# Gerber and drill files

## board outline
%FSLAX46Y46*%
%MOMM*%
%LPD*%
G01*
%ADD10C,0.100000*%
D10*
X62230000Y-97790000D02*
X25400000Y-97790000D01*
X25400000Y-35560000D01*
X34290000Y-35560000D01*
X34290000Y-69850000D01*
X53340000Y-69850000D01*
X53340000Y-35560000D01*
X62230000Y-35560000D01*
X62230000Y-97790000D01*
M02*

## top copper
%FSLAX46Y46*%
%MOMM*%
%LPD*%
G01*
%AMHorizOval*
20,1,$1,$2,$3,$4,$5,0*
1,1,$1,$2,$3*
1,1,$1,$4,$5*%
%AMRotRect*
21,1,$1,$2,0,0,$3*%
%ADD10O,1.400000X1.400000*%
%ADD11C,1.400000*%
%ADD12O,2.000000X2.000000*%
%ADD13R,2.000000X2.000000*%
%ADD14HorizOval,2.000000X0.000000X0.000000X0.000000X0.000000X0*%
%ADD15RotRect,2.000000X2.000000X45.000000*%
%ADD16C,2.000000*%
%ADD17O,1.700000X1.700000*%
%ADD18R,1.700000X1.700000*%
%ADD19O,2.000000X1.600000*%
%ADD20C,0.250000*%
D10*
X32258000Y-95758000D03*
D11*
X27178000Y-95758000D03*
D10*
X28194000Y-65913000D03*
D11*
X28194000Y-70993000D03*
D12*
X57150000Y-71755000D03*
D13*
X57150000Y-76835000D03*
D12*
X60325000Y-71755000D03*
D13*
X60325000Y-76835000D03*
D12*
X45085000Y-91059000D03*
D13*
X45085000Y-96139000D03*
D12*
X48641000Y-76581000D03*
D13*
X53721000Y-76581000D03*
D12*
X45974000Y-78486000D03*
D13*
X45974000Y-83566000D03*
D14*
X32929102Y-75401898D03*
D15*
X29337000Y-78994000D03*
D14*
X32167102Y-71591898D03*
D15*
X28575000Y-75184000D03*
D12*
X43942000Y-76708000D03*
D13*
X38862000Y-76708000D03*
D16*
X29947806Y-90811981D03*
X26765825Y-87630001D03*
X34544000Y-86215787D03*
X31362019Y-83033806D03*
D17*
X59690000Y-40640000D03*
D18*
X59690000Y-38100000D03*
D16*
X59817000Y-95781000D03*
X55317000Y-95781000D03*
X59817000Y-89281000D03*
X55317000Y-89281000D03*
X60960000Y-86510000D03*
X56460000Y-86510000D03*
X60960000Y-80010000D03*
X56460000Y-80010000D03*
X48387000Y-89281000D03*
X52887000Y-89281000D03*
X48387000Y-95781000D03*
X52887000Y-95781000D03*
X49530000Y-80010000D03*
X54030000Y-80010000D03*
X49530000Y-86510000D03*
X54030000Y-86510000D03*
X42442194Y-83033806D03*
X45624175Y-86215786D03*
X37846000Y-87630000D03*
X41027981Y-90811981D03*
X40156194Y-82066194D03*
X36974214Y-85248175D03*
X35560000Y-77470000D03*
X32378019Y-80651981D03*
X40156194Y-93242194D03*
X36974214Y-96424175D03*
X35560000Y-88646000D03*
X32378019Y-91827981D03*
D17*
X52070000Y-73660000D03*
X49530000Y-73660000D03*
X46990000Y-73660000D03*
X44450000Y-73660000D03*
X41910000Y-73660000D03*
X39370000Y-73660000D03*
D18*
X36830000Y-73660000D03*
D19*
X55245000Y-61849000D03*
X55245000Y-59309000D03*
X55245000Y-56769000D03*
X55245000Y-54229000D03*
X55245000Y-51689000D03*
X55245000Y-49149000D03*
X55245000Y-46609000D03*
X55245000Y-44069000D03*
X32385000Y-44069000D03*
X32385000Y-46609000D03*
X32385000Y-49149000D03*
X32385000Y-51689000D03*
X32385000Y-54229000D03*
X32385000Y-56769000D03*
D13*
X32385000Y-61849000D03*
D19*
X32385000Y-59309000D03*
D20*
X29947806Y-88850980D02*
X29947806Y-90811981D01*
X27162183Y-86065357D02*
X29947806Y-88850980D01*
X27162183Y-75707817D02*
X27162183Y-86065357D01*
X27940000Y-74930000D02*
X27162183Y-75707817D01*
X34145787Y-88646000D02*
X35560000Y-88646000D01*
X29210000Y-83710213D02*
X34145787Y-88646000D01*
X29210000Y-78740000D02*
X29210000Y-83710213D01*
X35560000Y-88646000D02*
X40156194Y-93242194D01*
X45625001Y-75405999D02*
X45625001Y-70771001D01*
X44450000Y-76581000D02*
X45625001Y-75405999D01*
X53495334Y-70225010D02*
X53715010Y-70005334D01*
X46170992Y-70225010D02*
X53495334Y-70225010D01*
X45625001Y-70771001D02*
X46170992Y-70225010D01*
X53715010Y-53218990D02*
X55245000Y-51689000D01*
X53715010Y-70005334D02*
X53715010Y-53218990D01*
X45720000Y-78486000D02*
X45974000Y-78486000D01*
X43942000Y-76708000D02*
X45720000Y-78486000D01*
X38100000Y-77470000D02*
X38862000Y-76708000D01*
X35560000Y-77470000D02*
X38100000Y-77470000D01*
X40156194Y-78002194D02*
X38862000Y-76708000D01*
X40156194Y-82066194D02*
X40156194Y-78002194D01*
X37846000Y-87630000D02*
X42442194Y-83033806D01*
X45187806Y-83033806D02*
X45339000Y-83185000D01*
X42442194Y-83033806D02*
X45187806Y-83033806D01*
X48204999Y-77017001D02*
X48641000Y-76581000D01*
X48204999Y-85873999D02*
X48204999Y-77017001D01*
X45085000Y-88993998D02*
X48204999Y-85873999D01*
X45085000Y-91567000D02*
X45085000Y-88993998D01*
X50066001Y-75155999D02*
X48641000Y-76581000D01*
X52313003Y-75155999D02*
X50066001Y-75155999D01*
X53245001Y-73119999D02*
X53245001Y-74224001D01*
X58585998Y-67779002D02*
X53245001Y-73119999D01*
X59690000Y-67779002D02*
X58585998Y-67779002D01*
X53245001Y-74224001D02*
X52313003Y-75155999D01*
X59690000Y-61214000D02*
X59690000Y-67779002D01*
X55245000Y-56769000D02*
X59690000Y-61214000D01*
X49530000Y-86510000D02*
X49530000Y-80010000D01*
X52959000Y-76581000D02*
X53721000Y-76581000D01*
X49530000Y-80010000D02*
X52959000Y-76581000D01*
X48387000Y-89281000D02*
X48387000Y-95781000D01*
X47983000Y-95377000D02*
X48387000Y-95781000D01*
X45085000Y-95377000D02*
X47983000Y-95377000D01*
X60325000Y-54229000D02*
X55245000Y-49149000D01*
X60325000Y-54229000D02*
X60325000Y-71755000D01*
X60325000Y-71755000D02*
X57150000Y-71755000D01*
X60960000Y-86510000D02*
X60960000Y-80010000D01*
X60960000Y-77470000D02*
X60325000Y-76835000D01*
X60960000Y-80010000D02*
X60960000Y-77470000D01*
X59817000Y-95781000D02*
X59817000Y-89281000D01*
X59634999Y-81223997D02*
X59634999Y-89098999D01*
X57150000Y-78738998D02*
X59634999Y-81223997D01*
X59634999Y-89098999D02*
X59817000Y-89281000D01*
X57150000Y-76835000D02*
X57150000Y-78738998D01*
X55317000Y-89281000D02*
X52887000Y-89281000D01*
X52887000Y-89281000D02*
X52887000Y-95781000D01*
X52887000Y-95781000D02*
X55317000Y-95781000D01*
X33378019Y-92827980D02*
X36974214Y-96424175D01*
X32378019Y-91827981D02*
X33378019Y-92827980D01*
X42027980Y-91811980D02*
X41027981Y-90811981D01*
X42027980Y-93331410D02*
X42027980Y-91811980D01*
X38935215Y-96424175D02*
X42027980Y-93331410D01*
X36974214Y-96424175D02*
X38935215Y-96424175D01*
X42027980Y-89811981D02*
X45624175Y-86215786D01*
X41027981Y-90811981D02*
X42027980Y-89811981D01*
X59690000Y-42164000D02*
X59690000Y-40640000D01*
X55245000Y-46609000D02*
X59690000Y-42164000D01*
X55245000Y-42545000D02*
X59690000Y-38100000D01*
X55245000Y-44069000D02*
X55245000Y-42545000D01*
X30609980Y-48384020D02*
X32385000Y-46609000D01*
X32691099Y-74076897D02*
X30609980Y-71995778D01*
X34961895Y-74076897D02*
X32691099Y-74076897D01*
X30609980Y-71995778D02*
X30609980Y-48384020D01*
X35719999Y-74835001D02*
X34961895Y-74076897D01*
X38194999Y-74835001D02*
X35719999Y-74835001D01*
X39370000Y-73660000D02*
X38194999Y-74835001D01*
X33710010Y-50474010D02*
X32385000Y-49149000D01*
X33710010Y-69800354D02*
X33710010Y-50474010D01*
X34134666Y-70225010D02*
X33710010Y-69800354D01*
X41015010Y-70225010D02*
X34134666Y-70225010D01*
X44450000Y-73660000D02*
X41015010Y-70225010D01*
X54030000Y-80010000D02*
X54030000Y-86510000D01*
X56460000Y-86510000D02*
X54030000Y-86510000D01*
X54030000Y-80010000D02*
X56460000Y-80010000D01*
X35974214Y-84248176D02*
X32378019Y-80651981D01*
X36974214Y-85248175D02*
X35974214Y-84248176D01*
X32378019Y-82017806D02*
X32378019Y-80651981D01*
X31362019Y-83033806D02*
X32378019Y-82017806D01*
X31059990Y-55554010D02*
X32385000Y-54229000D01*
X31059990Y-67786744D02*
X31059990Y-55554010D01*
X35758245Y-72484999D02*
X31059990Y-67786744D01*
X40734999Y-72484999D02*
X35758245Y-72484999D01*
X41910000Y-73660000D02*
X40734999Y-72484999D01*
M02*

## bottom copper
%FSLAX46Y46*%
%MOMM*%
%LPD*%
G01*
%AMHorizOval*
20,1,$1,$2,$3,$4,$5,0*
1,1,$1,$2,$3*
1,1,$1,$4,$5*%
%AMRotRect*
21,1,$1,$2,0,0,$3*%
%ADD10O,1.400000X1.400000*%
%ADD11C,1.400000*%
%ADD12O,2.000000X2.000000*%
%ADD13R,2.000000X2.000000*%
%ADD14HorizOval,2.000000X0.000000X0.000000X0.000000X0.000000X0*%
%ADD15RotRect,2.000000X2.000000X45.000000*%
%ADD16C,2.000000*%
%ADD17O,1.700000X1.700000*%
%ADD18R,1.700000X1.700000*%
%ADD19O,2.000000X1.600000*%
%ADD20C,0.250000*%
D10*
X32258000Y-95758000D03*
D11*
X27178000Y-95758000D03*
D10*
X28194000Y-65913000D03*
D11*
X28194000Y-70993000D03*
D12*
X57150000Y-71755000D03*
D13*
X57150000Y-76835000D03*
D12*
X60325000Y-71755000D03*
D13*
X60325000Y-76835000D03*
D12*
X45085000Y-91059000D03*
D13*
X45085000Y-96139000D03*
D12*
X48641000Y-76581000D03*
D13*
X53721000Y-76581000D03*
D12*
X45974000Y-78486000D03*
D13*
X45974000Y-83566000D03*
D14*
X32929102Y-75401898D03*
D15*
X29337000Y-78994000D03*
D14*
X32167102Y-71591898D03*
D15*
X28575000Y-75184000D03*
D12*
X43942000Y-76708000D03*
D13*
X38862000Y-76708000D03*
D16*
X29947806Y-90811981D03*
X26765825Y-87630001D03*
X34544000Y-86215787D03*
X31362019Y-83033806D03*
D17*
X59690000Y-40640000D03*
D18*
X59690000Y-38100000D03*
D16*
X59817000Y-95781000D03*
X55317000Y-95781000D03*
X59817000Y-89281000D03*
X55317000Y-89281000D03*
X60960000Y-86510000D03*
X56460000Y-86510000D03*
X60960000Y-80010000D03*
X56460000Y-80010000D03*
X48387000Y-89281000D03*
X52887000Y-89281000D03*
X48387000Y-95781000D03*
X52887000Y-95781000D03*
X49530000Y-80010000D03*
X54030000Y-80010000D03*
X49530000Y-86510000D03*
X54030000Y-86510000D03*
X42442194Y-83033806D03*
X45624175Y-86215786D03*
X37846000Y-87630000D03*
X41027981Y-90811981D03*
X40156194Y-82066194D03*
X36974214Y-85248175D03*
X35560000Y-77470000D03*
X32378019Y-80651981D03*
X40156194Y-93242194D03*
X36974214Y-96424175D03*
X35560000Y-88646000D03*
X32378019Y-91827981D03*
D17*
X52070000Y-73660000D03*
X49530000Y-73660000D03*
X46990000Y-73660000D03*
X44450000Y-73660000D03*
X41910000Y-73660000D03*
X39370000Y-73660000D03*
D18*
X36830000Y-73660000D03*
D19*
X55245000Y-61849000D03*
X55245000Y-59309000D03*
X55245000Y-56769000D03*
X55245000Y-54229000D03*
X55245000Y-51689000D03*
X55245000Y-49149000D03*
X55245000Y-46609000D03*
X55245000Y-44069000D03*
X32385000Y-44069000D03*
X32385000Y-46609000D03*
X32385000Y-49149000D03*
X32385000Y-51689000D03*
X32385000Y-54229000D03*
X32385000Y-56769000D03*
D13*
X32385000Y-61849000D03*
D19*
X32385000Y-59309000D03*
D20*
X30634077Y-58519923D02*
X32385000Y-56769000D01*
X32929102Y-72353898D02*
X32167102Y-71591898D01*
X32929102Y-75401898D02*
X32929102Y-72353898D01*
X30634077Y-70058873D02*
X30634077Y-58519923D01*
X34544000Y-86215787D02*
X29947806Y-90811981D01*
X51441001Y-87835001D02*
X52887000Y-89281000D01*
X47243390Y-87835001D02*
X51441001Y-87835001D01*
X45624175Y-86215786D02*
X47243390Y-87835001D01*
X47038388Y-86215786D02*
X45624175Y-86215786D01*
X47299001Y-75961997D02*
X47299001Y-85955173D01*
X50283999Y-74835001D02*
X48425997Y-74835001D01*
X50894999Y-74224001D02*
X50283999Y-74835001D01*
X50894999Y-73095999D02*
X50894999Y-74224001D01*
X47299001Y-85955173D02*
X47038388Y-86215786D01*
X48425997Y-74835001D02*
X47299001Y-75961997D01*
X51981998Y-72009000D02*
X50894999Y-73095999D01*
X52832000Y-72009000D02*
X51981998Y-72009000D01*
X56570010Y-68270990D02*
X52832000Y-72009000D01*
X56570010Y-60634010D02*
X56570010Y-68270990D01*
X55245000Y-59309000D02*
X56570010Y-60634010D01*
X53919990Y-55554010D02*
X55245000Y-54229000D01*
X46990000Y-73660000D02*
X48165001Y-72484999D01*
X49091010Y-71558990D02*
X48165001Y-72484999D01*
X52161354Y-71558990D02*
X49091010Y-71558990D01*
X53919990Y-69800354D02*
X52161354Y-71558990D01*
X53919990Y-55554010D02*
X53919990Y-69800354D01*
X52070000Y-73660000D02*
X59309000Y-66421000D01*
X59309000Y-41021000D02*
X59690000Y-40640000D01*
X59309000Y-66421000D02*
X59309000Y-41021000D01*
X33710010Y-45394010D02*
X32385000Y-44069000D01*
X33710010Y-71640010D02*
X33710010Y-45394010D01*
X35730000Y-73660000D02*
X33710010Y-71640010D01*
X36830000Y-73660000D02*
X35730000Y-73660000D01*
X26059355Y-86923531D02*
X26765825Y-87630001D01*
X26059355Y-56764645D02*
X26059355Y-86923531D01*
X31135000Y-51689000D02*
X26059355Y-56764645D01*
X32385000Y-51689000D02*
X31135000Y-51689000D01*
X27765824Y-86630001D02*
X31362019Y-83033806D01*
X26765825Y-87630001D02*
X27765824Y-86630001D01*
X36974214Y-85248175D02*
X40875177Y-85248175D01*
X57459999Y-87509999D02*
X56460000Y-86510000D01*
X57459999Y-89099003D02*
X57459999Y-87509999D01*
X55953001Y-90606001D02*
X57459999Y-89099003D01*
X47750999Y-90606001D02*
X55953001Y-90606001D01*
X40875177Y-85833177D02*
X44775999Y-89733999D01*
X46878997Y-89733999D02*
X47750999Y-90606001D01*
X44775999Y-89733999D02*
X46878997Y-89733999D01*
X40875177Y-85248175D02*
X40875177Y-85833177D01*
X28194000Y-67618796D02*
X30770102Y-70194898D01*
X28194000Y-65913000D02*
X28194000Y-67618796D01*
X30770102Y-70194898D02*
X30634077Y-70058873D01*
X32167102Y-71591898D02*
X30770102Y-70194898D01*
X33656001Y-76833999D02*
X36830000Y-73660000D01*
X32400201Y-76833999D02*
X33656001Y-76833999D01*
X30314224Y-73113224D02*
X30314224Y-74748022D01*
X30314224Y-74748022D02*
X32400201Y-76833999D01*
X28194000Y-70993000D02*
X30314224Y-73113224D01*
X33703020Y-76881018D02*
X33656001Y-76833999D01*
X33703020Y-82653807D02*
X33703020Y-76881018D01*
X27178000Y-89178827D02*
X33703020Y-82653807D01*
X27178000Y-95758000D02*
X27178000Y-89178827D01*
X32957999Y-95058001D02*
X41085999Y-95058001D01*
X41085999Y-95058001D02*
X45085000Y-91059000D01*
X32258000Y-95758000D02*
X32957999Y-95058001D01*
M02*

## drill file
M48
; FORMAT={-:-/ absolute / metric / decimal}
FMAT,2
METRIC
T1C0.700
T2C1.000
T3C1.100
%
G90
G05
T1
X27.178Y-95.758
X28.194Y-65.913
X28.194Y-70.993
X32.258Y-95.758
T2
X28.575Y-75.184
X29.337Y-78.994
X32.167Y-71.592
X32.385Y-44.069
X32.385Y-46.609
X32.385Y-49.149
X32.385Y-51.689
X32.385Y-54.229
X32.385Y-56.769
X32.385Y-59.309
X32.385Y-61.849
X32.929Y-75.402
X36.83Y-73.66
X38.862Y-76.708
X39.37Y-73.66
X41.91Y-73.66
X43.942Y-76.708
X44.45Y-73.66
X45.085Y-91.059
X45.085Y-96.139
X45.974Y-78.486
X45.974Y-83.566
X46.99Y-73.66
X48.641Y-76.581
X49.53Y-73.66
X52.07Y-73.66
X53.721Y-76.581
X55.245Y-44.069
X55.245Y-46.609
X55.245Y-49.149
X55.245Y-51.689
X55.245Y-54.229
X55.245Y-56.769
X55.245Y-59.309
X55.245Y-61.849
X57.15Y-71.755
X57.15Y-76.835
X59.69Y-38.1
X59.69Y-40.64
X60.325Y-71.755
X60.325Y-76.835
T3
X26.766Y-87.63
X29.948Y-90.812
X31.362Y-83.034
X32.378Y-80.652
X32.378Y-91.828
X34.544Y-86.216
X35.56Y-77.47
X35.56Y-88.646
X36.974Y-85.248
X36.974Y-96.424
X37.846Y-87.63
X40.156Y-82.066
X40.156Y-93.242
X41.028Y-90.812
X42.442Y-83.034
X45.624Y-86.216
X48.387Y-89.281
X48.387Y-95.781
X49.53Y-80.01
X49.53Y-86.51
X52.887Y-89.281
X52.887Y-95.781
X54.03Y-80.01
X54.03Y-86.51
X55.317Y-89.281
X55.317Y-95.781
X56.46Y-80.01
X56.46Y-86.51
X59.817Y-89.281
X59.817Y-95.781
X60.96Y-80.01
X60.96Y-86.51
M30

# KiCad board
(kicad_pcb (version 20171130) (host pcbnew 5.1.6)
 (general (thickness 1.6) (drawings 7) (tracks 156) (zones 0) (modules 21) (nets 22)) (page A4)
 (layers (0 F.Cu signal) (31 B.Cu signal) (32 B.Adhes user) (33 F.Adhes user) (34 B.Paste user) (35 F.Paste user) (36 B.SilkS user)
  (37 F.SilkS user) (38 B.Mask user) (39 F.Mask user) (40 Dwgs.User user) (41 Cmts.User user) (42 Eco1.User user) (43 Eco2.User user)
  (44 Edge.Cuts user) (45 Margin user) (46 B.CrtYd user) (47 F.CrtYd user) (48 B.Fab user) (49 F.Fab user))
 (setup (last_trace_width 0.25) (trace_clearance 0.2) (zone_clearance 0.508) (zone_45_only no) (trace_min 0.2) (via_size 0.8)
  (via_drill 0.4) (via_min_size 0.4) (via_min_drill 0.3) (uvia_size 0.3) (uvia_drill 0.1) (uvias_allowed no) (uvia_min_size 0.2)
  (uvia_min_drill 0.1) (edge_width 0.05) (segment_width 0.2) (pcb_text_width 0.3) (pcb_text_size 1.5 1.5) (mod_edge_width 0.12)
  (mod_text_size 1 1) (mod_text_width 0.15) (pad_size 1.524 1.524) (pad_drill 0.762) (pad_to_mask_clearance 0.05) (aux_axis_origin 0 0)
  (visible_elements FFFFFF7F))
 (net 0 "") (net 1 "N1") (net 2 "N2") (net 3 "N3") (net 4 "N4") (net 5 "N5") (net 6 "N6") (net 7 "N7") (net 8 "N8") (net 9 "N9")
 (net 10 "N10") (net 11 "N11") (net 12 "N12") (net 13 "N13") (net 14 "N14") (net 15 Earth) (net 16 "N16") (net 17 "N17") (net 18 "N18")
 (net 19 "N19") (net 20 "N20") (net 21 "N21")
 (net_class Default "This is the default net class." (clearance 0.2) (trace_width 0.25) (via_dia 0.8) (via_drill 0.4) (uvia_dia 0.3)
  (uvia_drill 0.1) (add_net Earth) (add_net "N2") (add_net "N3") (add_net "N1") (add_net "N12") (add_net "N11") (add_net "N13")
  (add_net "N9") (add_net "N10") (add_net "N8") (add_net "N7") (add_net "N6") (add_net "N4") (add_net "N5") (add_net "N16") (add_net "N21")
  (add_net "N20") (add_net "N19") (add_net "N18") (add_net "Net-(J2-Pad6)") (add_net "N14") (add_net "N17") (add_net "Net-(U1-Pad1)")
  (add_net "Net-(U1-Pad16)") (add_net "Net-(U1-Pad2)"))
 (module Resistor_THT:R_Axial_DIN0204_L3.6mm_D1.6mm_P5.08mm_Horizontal (layer F.Cu) (at 27.178 95.758)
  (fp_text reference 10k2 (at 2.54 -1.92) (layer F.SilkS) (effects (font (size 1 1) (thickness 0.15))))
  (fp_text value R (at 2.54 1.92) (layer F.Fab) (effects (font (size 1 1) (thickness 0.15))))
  (pad 2 thru_hole oval (at 5.08 0) (size 1.4 1.4) (drill 0.7) (layers *.Cu *.Mask) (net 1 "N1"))
  (pad 1 thru_hole circle (at 0 0) (size 1.4 1.4) (drill 0.7) (layers *.Cu *.Mask) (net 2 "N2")))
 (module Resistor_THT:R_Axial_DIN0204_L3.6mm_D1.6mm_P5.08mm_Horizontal (layer F.Cu) (at 28.194 70.993 90)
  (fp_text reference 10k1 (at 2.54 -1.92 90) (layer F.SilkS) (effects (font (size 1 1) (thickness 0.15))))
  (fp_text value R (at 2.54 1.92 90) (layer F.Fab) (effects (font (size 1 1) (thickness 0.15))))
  (pad 2 thru_hole oval (at 5.08 0 90) (size 1.4 1.4) (drill 0.7) (layers *.Cu *.Mask) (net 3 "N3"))
  (pad 1 thru_hole circle (at 0 0 90) (size 1.4 1.4) (drill 0.7) (layers *.Cu *.Mask) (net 2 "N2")))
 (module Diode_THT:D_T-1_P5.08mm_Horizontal (layer F.Cu) (at 57.15 76.835 90)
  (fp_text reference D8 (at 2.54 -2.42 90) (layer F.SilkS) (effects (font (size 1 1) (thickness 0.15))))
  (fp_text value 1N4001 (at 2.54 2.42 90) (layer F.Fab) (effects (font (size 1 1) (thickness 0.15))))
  (pad 2 thru_hole oval (at 5.08 0 90) (size 2 2) (drill 1) (layers *.Cu *.Mask) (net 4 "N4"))
  (pad 1 thru_hole rect (at 0 0 90) (size 2 2) (drill 1) (layers *.Cu *.Mask) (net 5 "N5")))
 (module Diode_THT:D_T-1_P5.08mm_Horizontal (layer F.Cu) (at 60.325 76.835 90)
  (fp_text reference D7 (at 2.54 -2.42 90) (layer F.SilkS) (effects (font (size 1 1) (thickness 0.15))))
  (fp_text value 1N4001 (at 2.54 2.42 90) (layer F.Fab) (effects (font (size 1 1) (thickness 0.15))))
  (pad 2 thru_hole oval (at 5.08 0 90) (size 2 2) (drill 1) (layers *.Cu *.Mask) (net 4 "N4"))
  (pad 1 thru_hole rect (at 0 0 90) (size 2 2) (drill 1) (layers *.Cu *.Mask) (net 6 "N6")))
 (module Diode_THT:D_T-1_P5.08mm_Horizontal (layer F.Cu) (at 45.085 96.139 90)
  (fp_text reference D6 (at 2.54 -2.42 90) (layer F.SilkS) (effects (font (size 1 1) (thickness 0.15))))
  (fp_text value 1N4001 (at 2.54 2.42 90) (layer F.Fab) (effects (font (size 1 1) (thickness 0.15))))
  (pad 2 thru_hole oval (at 5.08 0 90) (size 2 2) (drill 1) (layers *.Cu *.Mask) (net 1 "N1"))
  (pad 1 thru_hole rect (at 0 0 90) (size 2 2) (drill 1) (layers *.Cu *.Mask) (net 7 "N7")))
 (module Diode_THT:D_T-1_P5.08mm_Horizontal (layer F.Cu) (at 53.721 76.581 180)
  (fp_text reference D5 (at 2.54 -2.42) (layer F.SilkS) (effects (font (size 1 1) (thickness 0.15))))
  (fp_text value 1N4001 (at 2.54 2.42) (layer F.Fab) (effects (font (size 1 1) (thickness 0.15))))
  (pad 2 thru_hole oval (at 5.08 0 180) (size 2 2) (drill 1) (layers *.Cu *.Mask) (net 1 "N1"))
  (pad 1 thru_hole rect (at 0 0 180) (size 2 2) (drill 1) (layers *.Cu *.Mask) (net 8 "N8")))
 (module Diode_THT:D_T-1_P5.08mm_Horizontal (layer F.Cu) (at 45.974 83.566 90)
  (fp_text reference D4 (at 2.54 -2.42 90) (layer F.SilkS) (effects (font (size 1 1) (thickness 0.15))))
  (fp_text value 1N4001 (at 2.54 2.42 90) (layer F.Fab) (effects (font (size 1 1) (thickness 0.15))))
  (pad 2 thru_hole oval (at 5.08 0 90) (size 2 2) (drill 1) (layers *.Cu *.Mask) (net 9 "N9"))
  (pad 1 thru_hole rect (at 0 0 90) (size 2 2) (drill 1) (layers *.Cu *.Mask) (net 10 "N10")))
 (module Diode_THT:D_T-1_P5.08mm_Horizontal (layer F.Cu) (at 29.337 78.994 45)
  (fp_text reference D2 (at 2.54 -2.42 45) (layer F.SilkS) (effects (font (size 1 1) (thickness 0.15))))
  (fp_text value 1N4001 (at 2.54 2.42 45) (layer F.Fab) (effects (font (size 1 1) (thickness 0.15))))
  (pad 2 thru_hole oval (at 5.08 0 45) (size 2 2) (drill 1) (layers *.Cu *.Mask) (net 3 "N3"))
  (pad 1 thru_hole rect (at 0 0 45) (size 2 2) (drill 1) (layers *.Cu *.Mask) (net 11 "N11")))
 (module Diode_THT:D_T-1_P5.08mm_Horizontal (layer F.Cu) (at 28.575 75.184 45)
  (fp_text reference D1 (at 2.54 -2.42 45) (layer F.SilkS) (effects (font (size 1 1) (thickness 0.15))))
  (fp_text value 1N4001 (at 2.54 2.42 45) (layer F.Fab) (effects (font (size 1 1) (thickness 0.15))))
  (pad 2 thru_hole oval (at 5.08 0 45) (size 2 2) (drill 1) (layers *.Cu *.Mask) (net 3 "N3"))
  (pad 1 thru_hole rect (at 0 0 45) (size 2 2) (drill 1) (layers *.Cu *.Mask) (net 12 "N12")))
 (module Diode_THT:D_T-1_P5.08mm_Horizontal (layer F.Cu) (at 38.862 76.708)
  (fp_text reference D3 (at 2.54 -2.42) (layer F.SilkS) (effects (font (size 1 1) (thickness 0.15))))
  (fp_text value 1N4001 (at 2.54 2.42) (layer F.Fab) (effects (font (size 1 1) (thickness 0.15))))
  (pad 2 thru_hole oval (at 5.08 0) (size 2 2) (drill 1) (layers *.Cu *.Mask) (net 9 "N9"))
  (pad 1 thru_hole rect (at 0 0) (size 2 2) (drill 1) (layers *.Cu *.Mask) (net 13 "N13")))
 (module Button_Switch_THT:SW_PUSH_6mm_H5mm (layer F.Cu) (at 34.544 86.215787 225)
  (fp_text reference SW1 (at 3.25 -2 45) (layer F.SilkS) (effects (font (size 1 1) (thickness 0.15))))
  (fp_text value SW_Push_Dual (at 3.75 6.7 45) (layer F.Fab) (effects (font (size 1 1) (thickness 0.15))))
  (pad 1 thru_hole circle (at 6.5 0 315) (size 2 2) (drill 1.1) (layers *.Cu *.Mask) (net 12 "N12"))
  (pad 2 thru_hole circle (at 6.5 4.5 315) (size 2 2) (drill 1.1) (layers *.Cu *.Mask) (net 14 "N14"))
  (pad 1 thru_hole circle (at 0 0 315) (size 2 2) (drill 1.1) (layers *.Cu *.Mask) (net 12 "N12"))
  (pad 2 thru_hole circle (at 0 4.5 315) (size 2 2) (drill 1.1) (layers *.Cu *.Mask) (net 14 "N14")))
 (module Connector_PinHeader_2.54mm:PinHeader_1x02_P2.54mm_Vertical (layer F.Cu) (at 59.69 38.1)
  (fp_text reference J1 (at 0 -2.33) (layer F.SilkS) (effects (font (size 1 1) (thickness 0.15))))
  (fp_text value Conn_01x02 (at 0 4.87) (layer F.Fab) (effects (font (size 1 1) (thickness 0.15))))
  (pad 2 thru_hole oval (at 0 2.54) (size 1.7 1.7) (drill 1) (layers *.Cu *.Mask) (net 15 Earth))
  (pad 1 thru_hole rect (at 0 0) (size 1.7 1.7) (drill 1) (layers *.Cu *.Mask) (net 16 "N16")))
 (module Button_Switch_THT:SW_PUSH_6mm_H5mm (layer F.Cu) (at 59.817 89.281 270)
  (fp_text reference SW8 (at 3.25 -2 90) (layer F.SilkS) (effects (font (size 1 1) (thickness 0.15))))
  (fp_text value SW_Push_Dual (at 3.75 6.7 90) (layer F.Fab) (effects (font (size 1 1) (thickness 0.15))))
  (pad 1 thru_hole circle (at 6.5 0) (size 2 2) (drill 1.1) (layers *.Cu *.Mask) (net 5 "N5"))
  (pad 2 thru_hole circle (at 6.5 4.5) (size 2 2) (drill 1.1) (layers *.Cu *.Mask) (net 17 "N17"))
  (pad 1 thru_hole circle (at 0 0) (size 2 2) (drill 1.1) (layers *.Cu *.Mask) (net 5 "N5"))
  (pad 2 thru_hole circle (at 0 4.5) (size 2 2) (drill 1.1) (layers *.Cu *.Mask) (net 17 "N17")))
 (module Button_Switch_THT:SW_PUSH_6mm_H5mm (layer F.Cu) (at 60.96 80.01 270)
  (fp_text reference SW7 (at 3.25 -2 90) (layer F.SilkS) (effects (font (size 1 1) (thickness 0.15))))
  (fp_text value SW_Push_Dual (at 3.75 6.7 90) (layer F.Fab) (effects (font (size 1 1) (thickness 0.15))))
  (pad 1 thru_hole circle (at 6.5 0) (size 2 2) (drill 1.1) (layers *.Cu *.Mask) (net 6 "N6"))
  (pad 2 thru_hole circle (at 6.5 4.5) (size 2 2) (drill 1.1) (layers *.Cu *.Mask) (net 14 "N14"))
  (pad 1 thru_hole circle (at 0 0) (size 2 2) (drill 1.1) (layers *.Cu *.Mask) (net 6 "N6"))
  (pad 2 thru_hole circle (at 0 4.5) (size 2 2) (drill 1.1) (layers *.Cu *.Mask) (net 14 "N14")))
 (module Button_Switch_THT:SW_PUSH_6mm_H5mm (layer F.Cu) (at 48.387 95.781 90)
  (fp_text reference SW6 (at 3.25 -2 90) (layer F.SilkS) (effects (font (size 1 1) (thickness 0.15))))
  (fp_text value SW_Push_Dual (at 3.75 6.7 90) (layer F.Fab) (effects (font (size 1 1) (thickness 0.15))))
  (pad 1 thru_hole circle (at 6.5 0 180) (size 2 2) (drill 1.1) (layers *.Cu *.Mask) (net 7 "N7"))
  (pad 2 thru_hole circle (at 6.5 4.5 180) (size 2 2) (drill 1.1) (layers *.Cu *.Mask) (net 17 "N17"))
  (pad 1 thru_hole circle (at 0 0 180) (size 2 2) (drill 1.1) (layers *.Cu *.Mask) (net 7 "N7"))
  (pad 2 thru_hole circle (at 0 4.5 180) (size 2 2) (drill 1.1) (layers *.Cu *.Mask) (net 17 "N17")))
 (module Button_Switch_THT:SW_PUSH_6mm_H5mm (layer F.Cu) (at 49.53 86.51 90)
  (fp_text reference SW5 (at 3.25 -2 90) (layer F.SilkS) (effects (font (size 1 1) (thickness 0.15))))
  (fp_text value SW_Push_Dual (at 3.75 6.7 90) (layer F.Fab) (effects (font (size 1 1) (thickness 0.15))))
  (pad 1 thru_hole circle (at 6.5 0 180) (size 2 2) (drill 1.1) (layers *.Cu *.Mask) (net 8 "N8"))
  (pad 2 thru_hole circle (at 6.5 4.5 180) (size 2 2) (drill 1.1) (layers *.Cu *.Mask) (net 14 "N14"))
  (pad 1 thru_hole circle (at 0 0 180) (size 2 2) (drill 1.1) (layers *.Cu *.Mask) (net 8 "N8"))
  (pad 2 thru_hole circle (at 0 4.5 180) (size 2 2) (drill 1.1) (layers *.Cu *.Mask) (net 14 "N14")))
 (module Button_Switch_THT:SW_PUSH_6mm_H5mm (layer F.Cu) (at 37.846 87.63 45)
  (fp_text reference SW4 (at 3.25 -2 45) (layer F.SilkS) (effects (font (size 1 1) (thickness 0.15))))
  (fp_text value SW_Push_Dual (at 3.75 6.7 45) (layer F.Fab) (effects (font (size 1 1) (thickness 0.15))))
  (pad 1 thru_hole circle (at 6.5 0 135) (size 2 2) (drill 1.1) (layers *.Cu *.Mask) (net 10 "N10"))
  (pad 2 thru_hole circle (at 6.5 4.5 135) (size 2 2) (drill 1.1) (layers *.Cu *.Mask) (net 17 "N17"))
  (pad 1 thru_hole circle (at 0 0 135) (size 2 2) (drill 1.1) (layers *.Cu *.Mask) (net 10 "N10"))
  (pad 2 thru_hole circle (at 0 4.5 135) (size 2 2) (drill 1.1) (layers *.Cu *.Mask) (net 17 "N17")))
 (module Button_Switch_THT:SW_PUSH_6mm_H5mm (layer F.Cu) (at 35.56 77.47 315)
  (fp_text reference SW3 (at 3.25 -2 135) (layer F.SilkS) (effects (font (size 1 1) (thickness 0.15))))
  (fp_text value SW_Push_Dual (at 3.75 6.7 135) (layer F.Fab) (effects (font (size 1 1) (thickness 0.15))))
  (pad 1 thru_hole circle (at 6.5 0 45) (size 2 2) (drill 1.1) (layers *.Cu *.Mask) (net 13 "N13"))
  (pad 2 thru_hole circle (at 6.5 4.5 45) (size 2 2) (drill 1.1) (layers *.Cu *.Mask) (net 14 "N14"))
  (pad 1 thru_hole circle (at 0 0 45) (size 2 2) (drill 1.1) (layers *.Cu *.Mask) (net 13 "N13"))
  (pad 2 thru_hole circle (at 0 4.5 45) (size 2 2) (drill 1.1) (layers *.Cu *.Mask) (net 14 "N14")))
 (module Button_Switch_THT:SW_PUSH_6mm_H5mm (layer F.Cu) (at 35.56 88.646 315)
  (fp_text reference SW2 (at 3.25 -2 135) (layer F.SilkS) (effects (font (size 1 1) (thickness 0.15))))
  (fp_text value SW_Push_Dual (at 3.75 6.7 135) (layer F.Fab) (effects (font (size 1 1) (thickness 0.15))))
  (pad 1 thru_hole circle (at 6.5 0 45) (size 2 2) (drill 1.1) (layers *.Cu *.Mask) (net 11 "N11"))
  (pad 2 thru_hole circle (at 6.5 4.5 45) (size 2 2) (drill 1.1) (layers *.Cu *.Mask) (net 17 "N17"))
  (pad 1 thru_hole circle (at 0 0 45) (size 2 2) (drill 1.1) (layers *.Cu *.Mask) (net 11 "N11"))
  (pad 2 thru_hole circle (at 0 4.5 45) (size 2 2) (drill 1.1) (layers *.Cu *.Mask) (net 17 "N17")))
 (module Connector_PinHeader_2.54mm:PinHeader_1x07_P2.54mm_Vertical (layer F.Cu) (at 36.83 73.66 90)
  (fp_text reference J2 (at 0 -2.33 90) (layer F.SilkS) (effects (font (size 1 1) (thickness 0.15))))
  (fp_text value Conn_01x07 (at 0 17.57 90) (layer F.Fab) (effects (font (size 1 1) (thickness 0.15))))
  (pad 7 thru_hole oval (at 0 15.24 90) (size 1.7 1.7) (drill 1) (layers *.Cu *.Mask) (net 15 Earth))
  (pad 6 thru_hole oval (at 0 12.7 90) (size 1.7 1.7) (drill 1) (layers *.Cu *.Mask))
  (pad 5 thru_hole oval (at 0 10.16 90) (size 1.7 1.7) (drill 1) (layers *.Cu *.Mask) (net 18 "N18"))
  (pad 4 thru_hole oval (at 0 7.62 90) (size 1.7 1.7) (drill 1) (layers *.Cu *.Mask) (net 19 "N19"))
  (pad 3 thru_hole oval (at 0 5.08 90) (size 1.7 1.7) (drill 1) (layers *.Cu *.Mask) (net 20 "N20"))
  (pad 2 thru_hole oval (at 0 2.54 90) (size 1.7 1.7) (drill 1) (layers *.Cu *.Mask) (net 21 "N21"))
  (pad 1 thru_hole rect (at 0 0 90) (size 1.7 1.7) (drill 1) (layers *.Cu *.Mask) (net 2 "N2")))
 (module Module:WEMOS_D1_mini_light (layer B.Cu) (at 32.385 61.849)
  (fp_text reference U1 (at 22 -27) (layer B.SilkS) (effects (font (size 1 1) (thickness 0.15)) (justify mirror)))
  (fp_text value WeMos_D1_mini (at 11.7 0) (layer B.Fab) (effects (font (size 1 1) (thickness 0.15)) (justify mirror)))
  (pad 16 thru_hole oval (at 22.86 0) (size 2 1.6) (drill 1) (layers *.Cu *.Mask))
  (pad 15 thru_hole oval (at 22.86 -2.54) (size 2 1.6) (drill 1) (layers *.Cu *.Mask) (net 17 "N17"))
  (pad 14 thru_hole oval (at 22.86 -5.08) (size 2 1.6) (drill 1) (layers *.Cu *.Mask) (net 1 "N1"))
  (pad 13 thru_hole oval (at 22.86 -7.62) (size 2 1.6) (drill 1) (layers *.Cu *.Mask) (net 18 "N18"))
  (pad 12 thru_hole oval (at 22.86 -10.16) (size 2 1.6) (drill 1) (layers *.Cu *.Mask) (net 9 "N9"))
  (pad 11 thru_hole oval (at 22.86 -12.7) (size 2 1.6) (drill 1) (layers *.Cu *.Mask) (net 4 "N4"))
  (pad 10 thru_hole oval (at 22.86 -15.24) (size 2 1.6) (drill 1) (layers *.Cu *.Mask) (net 15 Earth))
  (pad 9 thru_hole oval (at 22.86 -17.78) (size 2 1.6) (drill 1) (layers *.Cu *.Mask) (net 16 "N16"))
  (pad 8 thru_hole oval (at 0 -17.78) (size 2 1.6) (drill 1) (layers *.Cu *.Mask) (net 2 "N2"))
  (pad 7 thru_hole oval (at 0 -15.24) (size 2 1.6) (drill 1) (layers *.Cu *.Mask) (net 21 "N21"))
  (pad 6 thru_hole oval (at 0 -12.7) (size 2 1.6) (drill 1) (layers *.Cu *.Mask) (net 19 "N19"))
  (pad 5 thru_hole oval (at 0 -10.16) (size 2 1.6) (drill 1) (layers *.Cu *.Mask) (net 14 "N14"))
  (pad 4 thru_hole oval (at 0 -7.62) (size 2 1.6) (drill 1) (layers *.Cu *.Mask) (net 20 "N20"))
  (pad 3 thru_hole oval (at 0 -5.08) (size 2 1.6) (drill 1) (layers *.Cu *.Mask) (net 3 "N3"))
  (pad 1 thru_hole rect (at 0 0) (size 2 2) (drill 1) (layers *.Cu *.Mask))
  (pad 2 thru_hole oval (at 0 -2.54) (size 2 1.6) (drill 1) (layers *.Cu *.Mask)))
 (gr_poly
  (pts (xy 62.23 97.79) (xy 25.4 97.79) (xy 25.4 35.56) (xy 34.29 35.56) (xy 34.29 69.85) (xy 53.34 69.85) (xy 53.34 35.56) (xy 62.23 35.56))
  (layer Edge.Cuts) (width 0.1))
 (segment (start 30.634077 58.519923) (end 32.385 56.769) (width 0.25) (layer B.Cu) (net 3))
 (segment (start 32.929102 72.353898) (end 32.167102 71.591898) (width 0.25) (layer B.Cu) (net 3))
 (segment (start 32.929102 75.401898) (end 32.929102 72.353898) (width 0.25) (layer B.Cu) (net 3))
 (segment (start 30.634077 70.058873) (end 30.634077 58.519923) (width 0.25) (layer B.Cu) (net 3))
 (segment (start 29.947806 88.85098) (end 29.947806 90.811981) (width 0.25) (layer F.Cu) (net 12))
 (segment (start 27.162183 86.065357) (end 29.947806 88.85098) (width 0.25) (layer F.Cu) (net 12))
 (segment (start 27.162183 75.707817) (end 27.162183 86.065357) (width 0.25) (layer F.Cu) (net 12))
 (segment (start 27.94 74.93) (end 27.162183 75.707817) (width 0.25) (layer F.Cu) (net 12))
 (segment (start 34.544 86.215787) (end 29.947806 90.811981) (width 0.25) (layer B.Cu) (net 12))
 (segment (start 34.145787 88.646) (end 35.56 88.646) (width 0.25) (layer F.Cu) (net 11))
 (segment (start 29.21 83.710213) (end 34.145787 88.646) (width 0.25) (layer F.Cu) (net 11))
 (segment (start 29.21 78.74) (end 29.21 83.710213) (width 0.25) (layer F.Cu) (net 11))
 (segment (start 35.56 88.646) (end 40.156194 93.242194) (width 0.25) (layer F.Cu) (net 11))
 (segment (start 45.625001 75.405999) (end 45.625001 70.771001) (width 0.25) (layer F.Cu) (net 9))
 (segment (start 44.45 76.581) (end 45.625001 75.405999) (width 0.25) (layer F.Cu) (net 9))
 (segment (start 53.495334 70.22501) (end 53.71501 70.005334) (width 0.25) (layer F.Cu) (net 9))
 (segment (start 46.170992 70.22501) (end 53.495334 70.22501) (width 0.25) (layer F.Cu) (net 9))
 (segment (start 45.625001 70.771001) (end 46.170992 70.22501) (width 0.25) (layer F.Cu) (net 9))
 (segment (start 53.71501 53.21899) (end 55.245 51.689) (width 0.25) (layer F.Cu) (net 9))
 (segment (start 53.71501 70.005334) (end 53.71501 53.21899) (width 0.25) (layer F.Cu) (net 9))
 (segment (start 45.72 78.486) (end 45.974 78.486) (width 0.25) (layer F.Cu) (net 9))
 (segment (start 43.942 76.708) (end 45.72 78.486) (width 0.25) (layer F.Cu) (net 9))
 (segment (start 38.1 77.47) (end 38.862 76.708) (width 0.25) (layer F.Cu) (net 13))
 (segment (start 35.56 77.47) (end 38.1 77.47) (width 0.25) (layer F.Cu) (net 13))
 (segment (start 40.156194 78.002194) (end 38.862 76.708) (width 0.25) (layer F.Cu) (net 13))
 (segment (start 40.156194 82.066194) (end 40.156194 78.002194) (width 0.25) (layer F.Cu) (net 13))
 (segment (start 37.846 87.63) (end 42.442194 83.033806) (width 0.25) (layer F.Cu) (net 10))
 (segment (start 45.187806 83.033806) (end 45.339 83.185) (width 0.25) (layer F.Cu) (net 10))
 (segment (start 42.442194 83.033806) (end 45.187806 83.033806) (width 0.25) (layer F.Cu) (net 10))
 (segment (start 48.204999 77.017001) (end 48.641 76.581) (width 0.25) (layer F.Cu) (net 1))
 (segment (start 48.204999 85.873999) (end 48.204999 77.017001) (width 0.25) (layer F.Cu) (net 1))
 (segment (start 45.085 88.993998) (end 48.204999 85.873999) (width 0.25) (layer F.Cu) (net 1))
 (segment (start 45.085 91.567) (end 45.085 88.993998) (width 0.25) (layer F.Cu) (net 1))
 (segment (start 50.066001 75.155999) (end 48.641 76.581) (width 0.25) (layer F.Cu) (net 1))
 (segment (start 52.313003 75.155999) (end 50.066001 75.155999) (width 0.25) (layer F.Cu) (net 1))
 (segment (start 53.245001 73.119999) (end 53.245001 74.224001) (width 0.25) (layer F.Cu) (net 1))
 (segment (start 58.585998 67.779002) (end 53.245001 73.119999) (width 0.25) (layer F.Cu) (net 1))
 (segment (start 59.69 67.779002) (end 58.585998 67.779002) (width 0.25) (layer F.Cu) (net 1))
 (segment (start 53.245001 74.224001) (end 52.313003 75.155999) (width 0.25) (layer F.Cu) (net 1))
 (segment (start 59.69 61.214) (end 59.69 67.779002) (width 0.25) (layer F.Cu) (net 1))
 (segment (start 55.245 56.769) (end 59.69 61.214) (width 0.25) (layer F.Cu) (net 1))
 (segment (start 49.53 86.51) (end 49.53 80.01) (width 0.25) (layer F.Cu) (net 8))
 (segment (start 52.959 76.581) (end 53.721 76.581) (width 0.25) (layer F.Cu) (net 8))
 (segment (start 49.53 80.01) (end 52.959 76.581) (width 0.25) (layer F.Cu) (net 8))
 (segment (start 48.387 89.281) (end 48.387 95.781) (width 0.25) (layer F.Cu) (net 7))
 (segment (start 47.983 95.377) (end 48.387 95.781) (width 0.25) (layer F.Cu) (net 7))
 (segment (start 45.085 95.377) (end 47.983 95.377) (width 0.25) (layer F.Cu) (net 7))
 (segment (start 60.325 54.229) (end 55.245 49.149) (width 0.25) (layer F.Cu) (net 4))
 (segment (start 60.325 54.229) (end 60.325 71.755) (width 0.25) (layer F.Cu) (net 4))
 (segment (start 60.325 71.755) (end 57.15 71.755) (width 0.25) (layer F.Cu) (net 4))
 (segment (start 60.96 86.51) (end 60.96 80.01) (width 0.25) (layer F.Cu) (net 6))
 (segment (start 60.96 77.47) (end 60.325 76.835) (width 0.25) (layer F.Cu) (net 6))
 (segment (start 60.96 80.01) (end 60.96 77.47) (width 0.25) (layer F.Cu) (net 6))
 (segment (start 59.817 95.781) (end 59.817 89.281) (width 0.25) (layer F.Cu) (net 5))
 (segment (start 59.634999 81.223997) (end 59.634999 89.098999) (width 0.25) (layer F.Cu) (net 5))
 (segment (start 57.15 78.738998) (end 59.634999 81.223997) (width 0.25) (layer F.Cu) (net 5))
 (segment (start 59.634999 89.098999) (end 59.817 89.281) (width 0.25) (layer F.Cu) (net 5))
 (segment (start 57.15 76.835) (end 57.15 78.738998) (width 0.25) (layer F.Cu) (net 5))
 (segment (start 55.317 89.281) (end 52.887 89.281) (width 0.25) (layer F.Cu) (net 17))
 (segment (start 52.887 89.281) (end 52.887 95.781) (width 0.25) (layer F.Cu) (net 17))
 (segment (start 52.887 95.781) (end 55.317 95.781) (width 0.25) (layer F.Cu) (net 17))
 (segment (start 33.378019 92.82798) (end 36.974214 96.424175) (width 0.25) (layer F.Cu) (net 17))
 (segment (start 32.378019 91.827981) (end 33.378019 92.82798) (width 0.25) (layer F.Cu) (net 17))
 (segment (start 42.02798 91.81198) (end 41.027981 90.811981) (width 0.25) (layer F.Cu) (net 17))
 (segment (start 42.02798 93.33141) (end 42.02798 91.81198) (width 0.25) (layer F.Cu) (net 17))
 (segment (start 38.935215 96.424175) (end 42.02798 93.33141) (width 0.25) (layer F.Cu) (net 17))
 (segment (start 36.974214 96.424175) (end 38.935215 96.424175) (width 0.25) (layer F.Cu) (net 17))
 (segment (start 42.02798 89.811981) (end 45.624175 86.215786) (width 0.25) (layer F.Cu) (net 17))
 (segment (start 41.027981 90.811981) (end 42.02798 89.811981) (width 0.25) (layer F.Cu) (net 17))
 (segment (start 51.441001 87.835001) (end 52.887 89.281) (width 0.25) (layer B.Cu) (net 17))
 (segment (start 47.24339 87.835001) (end 51.441001 87.835001) (width 0.25) (layer B.Cu) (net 17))
 (segment (start 45.624175 86.215786) (end 47.24339 87.835001) (width 0.25) (layer B.Cu) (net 17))
 (segment (start 47.038388 86.215786) (end 45.624175 86.215786) (width 0.25) (layer B.Cu) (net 17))
 (segment (start 47.299001 75.961997) (end 47.299001 85.955173) (width 0.25) (layer B.Cu) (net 17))
 (segment (start 50.283999 74.835001) (end 48.425997 74.835001) (width 0.25) (layer B.Cu) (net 17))
 (segment (start 50.894999 74.224001) (end 50.283999 74.835001) (width 0.25) (layer B.Cu) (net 17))
 (segment (start 50.894999 73.095999) (end 50.894999 74.224001) (width 0.25) (layer B.Cu) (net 17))
 (segment (start 47.299001 85.955173) (end 47.038388 86.215786) (width 0.25) (layer B.Cu) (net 17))
 (segment (start 48.425997 74.835001) (end 47.299001 75.961997) (width 0.25) (layer B.Cu) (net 17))
 (segment (start 51.981998 72.009) (end 50.894999 73.095999) (width 0.25) (layer B.Cu) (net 17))
 (segment (start 52.832 72.009) (end 51.981998 72.009) (width 0.25) (layer B.Cu) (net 17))
 (segment (start 56.57001 68.27099) (end 52.832 72.009) (width 0.25) (layer B.Cu) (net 17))
 (segment (start 56.57001 60.63401) (end 56.57001 68.27099) (width 0.25) (layer B.Cu) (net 17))
 (segment (start 55.245 59.309) (end 56.57001 60.63401) (width 0.25) (layer B.Cu) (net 17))
 (segment (start 53.91999 55.55401) (end 55.245 54.229) (width 0.25) (layer B.Cu) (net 18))
 (segment (start 46.99 73.66) (end 48.165001 72.484999) (width 0.25) (layer B.Cu) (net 18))
 (segment (start 49.09101 71.55899) (end 48.165001 72.484999) (width 0.25) (layer B.Cu) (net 18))
 (segment (start 52.161354 71.55899) (end 49.09101 71.55899) (width 0.25) (layer B.Cu) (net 18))
 (segment (start 53.91999 69.800354) (end 52.161354 71.55899) (width 0.25) (layer B.Cu) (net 18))
 (segment (start 53.91999 55.55401) (end 53.91999 69.800354) (width 0.25) (layer B.Cu) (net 18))
 (segment (start 59.69 42.164) (end 59.69 40.64) (width 0.25) (layer F.Cu) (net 15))
 (segment (start 55.245 46.609) (end 59.69 42.164) (width 0.25) (layer F.Cu) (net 15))
 (segment (start 52.07 73.66) (end 59.309 66.421) (width 0.25) (layer B.Cu) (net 15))
 (segment (start 59.309 41.021) (end 59.69 40.64) (width 0.25) (layer B.Cu) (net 15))
 (segment (start 59.309 66.421) (end 59.309 41.021) (width 0.25) (layer B.Cu) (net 15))
 (segment (start 55.245 42.545) (end 59.69 38.1) (width 0.25) (layer F.Cu) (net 16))
 (segment (start 55.245 44.069) (end 55.245 42.545) (width 0.25) (layer F.Cu) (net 16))
 (segment (start 33.71001 45.39401) (end 32.385 44.069) (width 0.25) (layer B.Cu) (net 2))
 (segment (start 33.71001 71.64001) (end 33.71001 45.39401) (width 0.25) (layer B.Cu) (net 2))
 (segment (start 35.73 73.66) (end 33.71001 71.64001) (width 0.25) (layer B.Cu) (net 2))
 (segment (start 36.83 73.66) (end 35.73 73.66) (width 0.25) (layer B.Cu) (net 2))
 (segment (start 30.60998 48.38402) (end 32.385 46.609) (width 0.25) (layer F.Cu) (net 21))
 (segment (start 32.691099 74.076897) (end 30.60998 71.995778) (width 0.25) (layer F.Cu) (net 21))
 (segment (start 34.961895 74.076897) (end 32.691099 74.076897) (width 0.25) (layer F.Cu) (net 21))
 (segment (start 30.60998 71.995778) (end 30.60998 48.38402) (width 0.25) (layer F.Cu) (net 21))
 (segment (start 35.719999 74.835001) (end 34.961895 74.076897) (width 0.25) (layer F.Cu) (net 21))
 (segment (start 38.194999 74.835001) (end 35.719999 74.835001) (width 0.25) (layer F.Cu) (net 21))
 (segment (start 39.37 73.66) (end 38.194999 74.835001) (width 0.25) (layer F.Cu) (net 21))
 (segment (start 33.71001 50.47401) (end 32.385 49.149) (width 0.25) (layer F.Cu) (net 19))
 (segment (start 33.71001 69.800354) (end 33.71001 50.47401) (width 0.25) (layer F.Cu) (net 19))
 (segment (start 34.134666 70.22501) (end 33.71001 69.800354) (width 0.25) (layer F.Cu) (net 19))
 (segment (start 41.01501 70.22501) (end 34.134666 70.22501) (width 0.25) (layer F.Cu) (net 19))
 (segment (start 44.45 73.66) (end 41.01501 70.22501) (width 0.25) (layer F.Cu) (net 19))
 (segment (start 54.03 80.01) (end 54.03 86.51) (width 0.25) (layer F.Cu) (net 14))
 (segment (start 56.46 86.51) (end 54.03 86.51) (width 0.25) (layer F.Cu) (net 14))
 (segment (start 54.03 80.01) (end 56.46 80.01) (width 0.25) (layer F.Cu) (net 14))
 (segment (start 26.059355 86.923531) (end 26.765825 87.630001) (width 0.25) (layer B.Cu) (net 14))
 (segment (start 26.059355 56.764645) (end 26.059355 86.923531) (width 0.25) (layer B.Cu) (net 14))
 (segment (start 31.135 51.689) (end 26.059355 56.764645) (width 0.25) (layer B.Cu) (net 14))
 (segment (start 32.385 51.689) (end 31.135 51.689) (width 0.25) (layer B.Cu) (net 14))
 (segment (start 27.765824 86.630001) (end 31.362019 83.033806) (width 0.25) (layer B.Cu) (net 14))
 (segment (start 26.765825 87.630001) (end 27.765824 86.630001) (width 0.25) (layer B.Cu) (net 14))
 (segment (start 36.974214 85.248175) (end 40.875177 85.248175) (width 0.25) (layer B.Cu) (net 14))
 (segment (start 57.459999 87.509999) (end 56.46 86.51) (width 0.25) (layer B.Cu) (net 14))
 (segment (start 57.459999 89.099003) (end 57.459999 87.509999) (width 0.25) (layer B.Cu) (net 14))
 (segment (start 55.953001 90.606001) (end 57.459999 89.099003) (width 0.25) (layer B.Cu) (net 14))
 (segment (start 47.750999 90.606001) (end 55.953001 90.606001) (width 0.25) (layer B.Cu) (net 14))
 (segment (start 40.875177 85.833177) (end 44.775999 89.733999) (width 0.25) (layer B.Cu) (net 14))
 (segment (start 46.878997 89.733999) (end 47.750999 90.606001) (width 0.25) (layer B.Cu) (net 14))
 (segment (start 44.775999 89.733999) (end 46.878997 89.733999) (width 0.25) (layer B.Cu) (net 14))
 (segment (start 40.875177 85.248175) (end 40.875177 85.833177) (width 0.25) (layer B.Cu) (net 14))
 (segment (start 35.974214 84.248176) (end 32.378019 80.651981) (width 0.25) (layer F.Cu) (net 14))
 (segment (start 36.974214 85.248175) (end 35.974214 84.248176) (width 0.25) (layer F.Cu) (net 14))
 (segment (start 32.378019 82.017806) (end 32.378019 80.651981) (width 0.25) (layer F.Cu) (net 14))
 (segment (start 31.362019 83.033806) (end 32.378019 82.017806) (width 0.25) (layer F.Cu) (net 14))
 (segment (start 31.05999 55.55401) (end 32.385 54.229) (width 0.25) (layer F.Cu) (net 20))
 (segment (start 31.05999 67.786744) (end 31.05999 55.55401) (width 0.25) (layer F.Cu) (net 20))
 (segment (start 35.758245 72.484999) (end 31.05999 67.786744) (width 0.25) (layer F.Cu) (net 20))
 (segment (start 40.734999 72.484999) (end 35.758245 72.484999) (width 0.25) (layer F.Cu) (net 20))
 (segment (start 41.91 73.66) (end 40.734999 72.484999) (width 0.25) (layer F.Cu) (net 20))
 (segment (start 28.194 67.618796) (end 30.770102 70.194898) (width 0.25) (layer B.Cu) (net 3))
 (segment (start 28.194 65.913) (end 28.194 67.618796) (width 0.25) (layer B.Cu) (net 3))
 (segment (start 30.770102 70.194898) (end 30.634077 70.058873) (width 0.25) (layer B.Cu) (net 3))
 (segment (start 32.167102 71.591898) (end 30.770102 70.194898) (width 0.25) (layer B.Cu) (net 3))
 (segment (start 33.656001 76.833999) (end 36.83 73.66) (width 0.25) (layer B.Cu) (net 2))
 (segment (start 32.400201 76.833999) (end 33.656001 76.833999) (width 0.25) (layer B.Cu) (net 2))
 (segment (start 30.314224 73.113224) (end 30.314224 74.748022) (width 0.25) (layer B.Cu) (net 2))
 (segment (start 30.314224 74.748022) (end 32.400201 76.833999) (width 0.25) (layer B.Cu) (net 2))
 (segment (start 28.194 70.993) (end 30.314224 73.113224) (width 0.25) (layer B.Cu) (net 2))
 (segment (start 33.70302 76.881018) (end 33.656001 76.833999) (width 0.25) (layer B.Cu) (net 2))
 (segment (start 33.70302 82.653807) (end 33.70302 76.881018) (width 0.25) (layer B.Cu) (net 2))
 (segment (start 27.178 89.178827) (end 33.70302 82.653807) (width 0.25) (layer B.Cu) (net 2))
 (segment (start 27.178 95.758) (end 27.178 89.178827) (width 0.25) (layer B.Cu) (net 2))
 (segment (start 32.957999 95.058001) (end 41.085999 95.058001) (width 0.25) (layer B.Cu) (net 1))
 (segment (start 41.085999 95.058001) (end 45.085 91.059) (width 0.25) (layer B.Cu) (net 1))
 (segment (start 32.258 95.758) (end 32.957999 95.058001) (width 0.25) (layer B.Cu) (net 1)))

